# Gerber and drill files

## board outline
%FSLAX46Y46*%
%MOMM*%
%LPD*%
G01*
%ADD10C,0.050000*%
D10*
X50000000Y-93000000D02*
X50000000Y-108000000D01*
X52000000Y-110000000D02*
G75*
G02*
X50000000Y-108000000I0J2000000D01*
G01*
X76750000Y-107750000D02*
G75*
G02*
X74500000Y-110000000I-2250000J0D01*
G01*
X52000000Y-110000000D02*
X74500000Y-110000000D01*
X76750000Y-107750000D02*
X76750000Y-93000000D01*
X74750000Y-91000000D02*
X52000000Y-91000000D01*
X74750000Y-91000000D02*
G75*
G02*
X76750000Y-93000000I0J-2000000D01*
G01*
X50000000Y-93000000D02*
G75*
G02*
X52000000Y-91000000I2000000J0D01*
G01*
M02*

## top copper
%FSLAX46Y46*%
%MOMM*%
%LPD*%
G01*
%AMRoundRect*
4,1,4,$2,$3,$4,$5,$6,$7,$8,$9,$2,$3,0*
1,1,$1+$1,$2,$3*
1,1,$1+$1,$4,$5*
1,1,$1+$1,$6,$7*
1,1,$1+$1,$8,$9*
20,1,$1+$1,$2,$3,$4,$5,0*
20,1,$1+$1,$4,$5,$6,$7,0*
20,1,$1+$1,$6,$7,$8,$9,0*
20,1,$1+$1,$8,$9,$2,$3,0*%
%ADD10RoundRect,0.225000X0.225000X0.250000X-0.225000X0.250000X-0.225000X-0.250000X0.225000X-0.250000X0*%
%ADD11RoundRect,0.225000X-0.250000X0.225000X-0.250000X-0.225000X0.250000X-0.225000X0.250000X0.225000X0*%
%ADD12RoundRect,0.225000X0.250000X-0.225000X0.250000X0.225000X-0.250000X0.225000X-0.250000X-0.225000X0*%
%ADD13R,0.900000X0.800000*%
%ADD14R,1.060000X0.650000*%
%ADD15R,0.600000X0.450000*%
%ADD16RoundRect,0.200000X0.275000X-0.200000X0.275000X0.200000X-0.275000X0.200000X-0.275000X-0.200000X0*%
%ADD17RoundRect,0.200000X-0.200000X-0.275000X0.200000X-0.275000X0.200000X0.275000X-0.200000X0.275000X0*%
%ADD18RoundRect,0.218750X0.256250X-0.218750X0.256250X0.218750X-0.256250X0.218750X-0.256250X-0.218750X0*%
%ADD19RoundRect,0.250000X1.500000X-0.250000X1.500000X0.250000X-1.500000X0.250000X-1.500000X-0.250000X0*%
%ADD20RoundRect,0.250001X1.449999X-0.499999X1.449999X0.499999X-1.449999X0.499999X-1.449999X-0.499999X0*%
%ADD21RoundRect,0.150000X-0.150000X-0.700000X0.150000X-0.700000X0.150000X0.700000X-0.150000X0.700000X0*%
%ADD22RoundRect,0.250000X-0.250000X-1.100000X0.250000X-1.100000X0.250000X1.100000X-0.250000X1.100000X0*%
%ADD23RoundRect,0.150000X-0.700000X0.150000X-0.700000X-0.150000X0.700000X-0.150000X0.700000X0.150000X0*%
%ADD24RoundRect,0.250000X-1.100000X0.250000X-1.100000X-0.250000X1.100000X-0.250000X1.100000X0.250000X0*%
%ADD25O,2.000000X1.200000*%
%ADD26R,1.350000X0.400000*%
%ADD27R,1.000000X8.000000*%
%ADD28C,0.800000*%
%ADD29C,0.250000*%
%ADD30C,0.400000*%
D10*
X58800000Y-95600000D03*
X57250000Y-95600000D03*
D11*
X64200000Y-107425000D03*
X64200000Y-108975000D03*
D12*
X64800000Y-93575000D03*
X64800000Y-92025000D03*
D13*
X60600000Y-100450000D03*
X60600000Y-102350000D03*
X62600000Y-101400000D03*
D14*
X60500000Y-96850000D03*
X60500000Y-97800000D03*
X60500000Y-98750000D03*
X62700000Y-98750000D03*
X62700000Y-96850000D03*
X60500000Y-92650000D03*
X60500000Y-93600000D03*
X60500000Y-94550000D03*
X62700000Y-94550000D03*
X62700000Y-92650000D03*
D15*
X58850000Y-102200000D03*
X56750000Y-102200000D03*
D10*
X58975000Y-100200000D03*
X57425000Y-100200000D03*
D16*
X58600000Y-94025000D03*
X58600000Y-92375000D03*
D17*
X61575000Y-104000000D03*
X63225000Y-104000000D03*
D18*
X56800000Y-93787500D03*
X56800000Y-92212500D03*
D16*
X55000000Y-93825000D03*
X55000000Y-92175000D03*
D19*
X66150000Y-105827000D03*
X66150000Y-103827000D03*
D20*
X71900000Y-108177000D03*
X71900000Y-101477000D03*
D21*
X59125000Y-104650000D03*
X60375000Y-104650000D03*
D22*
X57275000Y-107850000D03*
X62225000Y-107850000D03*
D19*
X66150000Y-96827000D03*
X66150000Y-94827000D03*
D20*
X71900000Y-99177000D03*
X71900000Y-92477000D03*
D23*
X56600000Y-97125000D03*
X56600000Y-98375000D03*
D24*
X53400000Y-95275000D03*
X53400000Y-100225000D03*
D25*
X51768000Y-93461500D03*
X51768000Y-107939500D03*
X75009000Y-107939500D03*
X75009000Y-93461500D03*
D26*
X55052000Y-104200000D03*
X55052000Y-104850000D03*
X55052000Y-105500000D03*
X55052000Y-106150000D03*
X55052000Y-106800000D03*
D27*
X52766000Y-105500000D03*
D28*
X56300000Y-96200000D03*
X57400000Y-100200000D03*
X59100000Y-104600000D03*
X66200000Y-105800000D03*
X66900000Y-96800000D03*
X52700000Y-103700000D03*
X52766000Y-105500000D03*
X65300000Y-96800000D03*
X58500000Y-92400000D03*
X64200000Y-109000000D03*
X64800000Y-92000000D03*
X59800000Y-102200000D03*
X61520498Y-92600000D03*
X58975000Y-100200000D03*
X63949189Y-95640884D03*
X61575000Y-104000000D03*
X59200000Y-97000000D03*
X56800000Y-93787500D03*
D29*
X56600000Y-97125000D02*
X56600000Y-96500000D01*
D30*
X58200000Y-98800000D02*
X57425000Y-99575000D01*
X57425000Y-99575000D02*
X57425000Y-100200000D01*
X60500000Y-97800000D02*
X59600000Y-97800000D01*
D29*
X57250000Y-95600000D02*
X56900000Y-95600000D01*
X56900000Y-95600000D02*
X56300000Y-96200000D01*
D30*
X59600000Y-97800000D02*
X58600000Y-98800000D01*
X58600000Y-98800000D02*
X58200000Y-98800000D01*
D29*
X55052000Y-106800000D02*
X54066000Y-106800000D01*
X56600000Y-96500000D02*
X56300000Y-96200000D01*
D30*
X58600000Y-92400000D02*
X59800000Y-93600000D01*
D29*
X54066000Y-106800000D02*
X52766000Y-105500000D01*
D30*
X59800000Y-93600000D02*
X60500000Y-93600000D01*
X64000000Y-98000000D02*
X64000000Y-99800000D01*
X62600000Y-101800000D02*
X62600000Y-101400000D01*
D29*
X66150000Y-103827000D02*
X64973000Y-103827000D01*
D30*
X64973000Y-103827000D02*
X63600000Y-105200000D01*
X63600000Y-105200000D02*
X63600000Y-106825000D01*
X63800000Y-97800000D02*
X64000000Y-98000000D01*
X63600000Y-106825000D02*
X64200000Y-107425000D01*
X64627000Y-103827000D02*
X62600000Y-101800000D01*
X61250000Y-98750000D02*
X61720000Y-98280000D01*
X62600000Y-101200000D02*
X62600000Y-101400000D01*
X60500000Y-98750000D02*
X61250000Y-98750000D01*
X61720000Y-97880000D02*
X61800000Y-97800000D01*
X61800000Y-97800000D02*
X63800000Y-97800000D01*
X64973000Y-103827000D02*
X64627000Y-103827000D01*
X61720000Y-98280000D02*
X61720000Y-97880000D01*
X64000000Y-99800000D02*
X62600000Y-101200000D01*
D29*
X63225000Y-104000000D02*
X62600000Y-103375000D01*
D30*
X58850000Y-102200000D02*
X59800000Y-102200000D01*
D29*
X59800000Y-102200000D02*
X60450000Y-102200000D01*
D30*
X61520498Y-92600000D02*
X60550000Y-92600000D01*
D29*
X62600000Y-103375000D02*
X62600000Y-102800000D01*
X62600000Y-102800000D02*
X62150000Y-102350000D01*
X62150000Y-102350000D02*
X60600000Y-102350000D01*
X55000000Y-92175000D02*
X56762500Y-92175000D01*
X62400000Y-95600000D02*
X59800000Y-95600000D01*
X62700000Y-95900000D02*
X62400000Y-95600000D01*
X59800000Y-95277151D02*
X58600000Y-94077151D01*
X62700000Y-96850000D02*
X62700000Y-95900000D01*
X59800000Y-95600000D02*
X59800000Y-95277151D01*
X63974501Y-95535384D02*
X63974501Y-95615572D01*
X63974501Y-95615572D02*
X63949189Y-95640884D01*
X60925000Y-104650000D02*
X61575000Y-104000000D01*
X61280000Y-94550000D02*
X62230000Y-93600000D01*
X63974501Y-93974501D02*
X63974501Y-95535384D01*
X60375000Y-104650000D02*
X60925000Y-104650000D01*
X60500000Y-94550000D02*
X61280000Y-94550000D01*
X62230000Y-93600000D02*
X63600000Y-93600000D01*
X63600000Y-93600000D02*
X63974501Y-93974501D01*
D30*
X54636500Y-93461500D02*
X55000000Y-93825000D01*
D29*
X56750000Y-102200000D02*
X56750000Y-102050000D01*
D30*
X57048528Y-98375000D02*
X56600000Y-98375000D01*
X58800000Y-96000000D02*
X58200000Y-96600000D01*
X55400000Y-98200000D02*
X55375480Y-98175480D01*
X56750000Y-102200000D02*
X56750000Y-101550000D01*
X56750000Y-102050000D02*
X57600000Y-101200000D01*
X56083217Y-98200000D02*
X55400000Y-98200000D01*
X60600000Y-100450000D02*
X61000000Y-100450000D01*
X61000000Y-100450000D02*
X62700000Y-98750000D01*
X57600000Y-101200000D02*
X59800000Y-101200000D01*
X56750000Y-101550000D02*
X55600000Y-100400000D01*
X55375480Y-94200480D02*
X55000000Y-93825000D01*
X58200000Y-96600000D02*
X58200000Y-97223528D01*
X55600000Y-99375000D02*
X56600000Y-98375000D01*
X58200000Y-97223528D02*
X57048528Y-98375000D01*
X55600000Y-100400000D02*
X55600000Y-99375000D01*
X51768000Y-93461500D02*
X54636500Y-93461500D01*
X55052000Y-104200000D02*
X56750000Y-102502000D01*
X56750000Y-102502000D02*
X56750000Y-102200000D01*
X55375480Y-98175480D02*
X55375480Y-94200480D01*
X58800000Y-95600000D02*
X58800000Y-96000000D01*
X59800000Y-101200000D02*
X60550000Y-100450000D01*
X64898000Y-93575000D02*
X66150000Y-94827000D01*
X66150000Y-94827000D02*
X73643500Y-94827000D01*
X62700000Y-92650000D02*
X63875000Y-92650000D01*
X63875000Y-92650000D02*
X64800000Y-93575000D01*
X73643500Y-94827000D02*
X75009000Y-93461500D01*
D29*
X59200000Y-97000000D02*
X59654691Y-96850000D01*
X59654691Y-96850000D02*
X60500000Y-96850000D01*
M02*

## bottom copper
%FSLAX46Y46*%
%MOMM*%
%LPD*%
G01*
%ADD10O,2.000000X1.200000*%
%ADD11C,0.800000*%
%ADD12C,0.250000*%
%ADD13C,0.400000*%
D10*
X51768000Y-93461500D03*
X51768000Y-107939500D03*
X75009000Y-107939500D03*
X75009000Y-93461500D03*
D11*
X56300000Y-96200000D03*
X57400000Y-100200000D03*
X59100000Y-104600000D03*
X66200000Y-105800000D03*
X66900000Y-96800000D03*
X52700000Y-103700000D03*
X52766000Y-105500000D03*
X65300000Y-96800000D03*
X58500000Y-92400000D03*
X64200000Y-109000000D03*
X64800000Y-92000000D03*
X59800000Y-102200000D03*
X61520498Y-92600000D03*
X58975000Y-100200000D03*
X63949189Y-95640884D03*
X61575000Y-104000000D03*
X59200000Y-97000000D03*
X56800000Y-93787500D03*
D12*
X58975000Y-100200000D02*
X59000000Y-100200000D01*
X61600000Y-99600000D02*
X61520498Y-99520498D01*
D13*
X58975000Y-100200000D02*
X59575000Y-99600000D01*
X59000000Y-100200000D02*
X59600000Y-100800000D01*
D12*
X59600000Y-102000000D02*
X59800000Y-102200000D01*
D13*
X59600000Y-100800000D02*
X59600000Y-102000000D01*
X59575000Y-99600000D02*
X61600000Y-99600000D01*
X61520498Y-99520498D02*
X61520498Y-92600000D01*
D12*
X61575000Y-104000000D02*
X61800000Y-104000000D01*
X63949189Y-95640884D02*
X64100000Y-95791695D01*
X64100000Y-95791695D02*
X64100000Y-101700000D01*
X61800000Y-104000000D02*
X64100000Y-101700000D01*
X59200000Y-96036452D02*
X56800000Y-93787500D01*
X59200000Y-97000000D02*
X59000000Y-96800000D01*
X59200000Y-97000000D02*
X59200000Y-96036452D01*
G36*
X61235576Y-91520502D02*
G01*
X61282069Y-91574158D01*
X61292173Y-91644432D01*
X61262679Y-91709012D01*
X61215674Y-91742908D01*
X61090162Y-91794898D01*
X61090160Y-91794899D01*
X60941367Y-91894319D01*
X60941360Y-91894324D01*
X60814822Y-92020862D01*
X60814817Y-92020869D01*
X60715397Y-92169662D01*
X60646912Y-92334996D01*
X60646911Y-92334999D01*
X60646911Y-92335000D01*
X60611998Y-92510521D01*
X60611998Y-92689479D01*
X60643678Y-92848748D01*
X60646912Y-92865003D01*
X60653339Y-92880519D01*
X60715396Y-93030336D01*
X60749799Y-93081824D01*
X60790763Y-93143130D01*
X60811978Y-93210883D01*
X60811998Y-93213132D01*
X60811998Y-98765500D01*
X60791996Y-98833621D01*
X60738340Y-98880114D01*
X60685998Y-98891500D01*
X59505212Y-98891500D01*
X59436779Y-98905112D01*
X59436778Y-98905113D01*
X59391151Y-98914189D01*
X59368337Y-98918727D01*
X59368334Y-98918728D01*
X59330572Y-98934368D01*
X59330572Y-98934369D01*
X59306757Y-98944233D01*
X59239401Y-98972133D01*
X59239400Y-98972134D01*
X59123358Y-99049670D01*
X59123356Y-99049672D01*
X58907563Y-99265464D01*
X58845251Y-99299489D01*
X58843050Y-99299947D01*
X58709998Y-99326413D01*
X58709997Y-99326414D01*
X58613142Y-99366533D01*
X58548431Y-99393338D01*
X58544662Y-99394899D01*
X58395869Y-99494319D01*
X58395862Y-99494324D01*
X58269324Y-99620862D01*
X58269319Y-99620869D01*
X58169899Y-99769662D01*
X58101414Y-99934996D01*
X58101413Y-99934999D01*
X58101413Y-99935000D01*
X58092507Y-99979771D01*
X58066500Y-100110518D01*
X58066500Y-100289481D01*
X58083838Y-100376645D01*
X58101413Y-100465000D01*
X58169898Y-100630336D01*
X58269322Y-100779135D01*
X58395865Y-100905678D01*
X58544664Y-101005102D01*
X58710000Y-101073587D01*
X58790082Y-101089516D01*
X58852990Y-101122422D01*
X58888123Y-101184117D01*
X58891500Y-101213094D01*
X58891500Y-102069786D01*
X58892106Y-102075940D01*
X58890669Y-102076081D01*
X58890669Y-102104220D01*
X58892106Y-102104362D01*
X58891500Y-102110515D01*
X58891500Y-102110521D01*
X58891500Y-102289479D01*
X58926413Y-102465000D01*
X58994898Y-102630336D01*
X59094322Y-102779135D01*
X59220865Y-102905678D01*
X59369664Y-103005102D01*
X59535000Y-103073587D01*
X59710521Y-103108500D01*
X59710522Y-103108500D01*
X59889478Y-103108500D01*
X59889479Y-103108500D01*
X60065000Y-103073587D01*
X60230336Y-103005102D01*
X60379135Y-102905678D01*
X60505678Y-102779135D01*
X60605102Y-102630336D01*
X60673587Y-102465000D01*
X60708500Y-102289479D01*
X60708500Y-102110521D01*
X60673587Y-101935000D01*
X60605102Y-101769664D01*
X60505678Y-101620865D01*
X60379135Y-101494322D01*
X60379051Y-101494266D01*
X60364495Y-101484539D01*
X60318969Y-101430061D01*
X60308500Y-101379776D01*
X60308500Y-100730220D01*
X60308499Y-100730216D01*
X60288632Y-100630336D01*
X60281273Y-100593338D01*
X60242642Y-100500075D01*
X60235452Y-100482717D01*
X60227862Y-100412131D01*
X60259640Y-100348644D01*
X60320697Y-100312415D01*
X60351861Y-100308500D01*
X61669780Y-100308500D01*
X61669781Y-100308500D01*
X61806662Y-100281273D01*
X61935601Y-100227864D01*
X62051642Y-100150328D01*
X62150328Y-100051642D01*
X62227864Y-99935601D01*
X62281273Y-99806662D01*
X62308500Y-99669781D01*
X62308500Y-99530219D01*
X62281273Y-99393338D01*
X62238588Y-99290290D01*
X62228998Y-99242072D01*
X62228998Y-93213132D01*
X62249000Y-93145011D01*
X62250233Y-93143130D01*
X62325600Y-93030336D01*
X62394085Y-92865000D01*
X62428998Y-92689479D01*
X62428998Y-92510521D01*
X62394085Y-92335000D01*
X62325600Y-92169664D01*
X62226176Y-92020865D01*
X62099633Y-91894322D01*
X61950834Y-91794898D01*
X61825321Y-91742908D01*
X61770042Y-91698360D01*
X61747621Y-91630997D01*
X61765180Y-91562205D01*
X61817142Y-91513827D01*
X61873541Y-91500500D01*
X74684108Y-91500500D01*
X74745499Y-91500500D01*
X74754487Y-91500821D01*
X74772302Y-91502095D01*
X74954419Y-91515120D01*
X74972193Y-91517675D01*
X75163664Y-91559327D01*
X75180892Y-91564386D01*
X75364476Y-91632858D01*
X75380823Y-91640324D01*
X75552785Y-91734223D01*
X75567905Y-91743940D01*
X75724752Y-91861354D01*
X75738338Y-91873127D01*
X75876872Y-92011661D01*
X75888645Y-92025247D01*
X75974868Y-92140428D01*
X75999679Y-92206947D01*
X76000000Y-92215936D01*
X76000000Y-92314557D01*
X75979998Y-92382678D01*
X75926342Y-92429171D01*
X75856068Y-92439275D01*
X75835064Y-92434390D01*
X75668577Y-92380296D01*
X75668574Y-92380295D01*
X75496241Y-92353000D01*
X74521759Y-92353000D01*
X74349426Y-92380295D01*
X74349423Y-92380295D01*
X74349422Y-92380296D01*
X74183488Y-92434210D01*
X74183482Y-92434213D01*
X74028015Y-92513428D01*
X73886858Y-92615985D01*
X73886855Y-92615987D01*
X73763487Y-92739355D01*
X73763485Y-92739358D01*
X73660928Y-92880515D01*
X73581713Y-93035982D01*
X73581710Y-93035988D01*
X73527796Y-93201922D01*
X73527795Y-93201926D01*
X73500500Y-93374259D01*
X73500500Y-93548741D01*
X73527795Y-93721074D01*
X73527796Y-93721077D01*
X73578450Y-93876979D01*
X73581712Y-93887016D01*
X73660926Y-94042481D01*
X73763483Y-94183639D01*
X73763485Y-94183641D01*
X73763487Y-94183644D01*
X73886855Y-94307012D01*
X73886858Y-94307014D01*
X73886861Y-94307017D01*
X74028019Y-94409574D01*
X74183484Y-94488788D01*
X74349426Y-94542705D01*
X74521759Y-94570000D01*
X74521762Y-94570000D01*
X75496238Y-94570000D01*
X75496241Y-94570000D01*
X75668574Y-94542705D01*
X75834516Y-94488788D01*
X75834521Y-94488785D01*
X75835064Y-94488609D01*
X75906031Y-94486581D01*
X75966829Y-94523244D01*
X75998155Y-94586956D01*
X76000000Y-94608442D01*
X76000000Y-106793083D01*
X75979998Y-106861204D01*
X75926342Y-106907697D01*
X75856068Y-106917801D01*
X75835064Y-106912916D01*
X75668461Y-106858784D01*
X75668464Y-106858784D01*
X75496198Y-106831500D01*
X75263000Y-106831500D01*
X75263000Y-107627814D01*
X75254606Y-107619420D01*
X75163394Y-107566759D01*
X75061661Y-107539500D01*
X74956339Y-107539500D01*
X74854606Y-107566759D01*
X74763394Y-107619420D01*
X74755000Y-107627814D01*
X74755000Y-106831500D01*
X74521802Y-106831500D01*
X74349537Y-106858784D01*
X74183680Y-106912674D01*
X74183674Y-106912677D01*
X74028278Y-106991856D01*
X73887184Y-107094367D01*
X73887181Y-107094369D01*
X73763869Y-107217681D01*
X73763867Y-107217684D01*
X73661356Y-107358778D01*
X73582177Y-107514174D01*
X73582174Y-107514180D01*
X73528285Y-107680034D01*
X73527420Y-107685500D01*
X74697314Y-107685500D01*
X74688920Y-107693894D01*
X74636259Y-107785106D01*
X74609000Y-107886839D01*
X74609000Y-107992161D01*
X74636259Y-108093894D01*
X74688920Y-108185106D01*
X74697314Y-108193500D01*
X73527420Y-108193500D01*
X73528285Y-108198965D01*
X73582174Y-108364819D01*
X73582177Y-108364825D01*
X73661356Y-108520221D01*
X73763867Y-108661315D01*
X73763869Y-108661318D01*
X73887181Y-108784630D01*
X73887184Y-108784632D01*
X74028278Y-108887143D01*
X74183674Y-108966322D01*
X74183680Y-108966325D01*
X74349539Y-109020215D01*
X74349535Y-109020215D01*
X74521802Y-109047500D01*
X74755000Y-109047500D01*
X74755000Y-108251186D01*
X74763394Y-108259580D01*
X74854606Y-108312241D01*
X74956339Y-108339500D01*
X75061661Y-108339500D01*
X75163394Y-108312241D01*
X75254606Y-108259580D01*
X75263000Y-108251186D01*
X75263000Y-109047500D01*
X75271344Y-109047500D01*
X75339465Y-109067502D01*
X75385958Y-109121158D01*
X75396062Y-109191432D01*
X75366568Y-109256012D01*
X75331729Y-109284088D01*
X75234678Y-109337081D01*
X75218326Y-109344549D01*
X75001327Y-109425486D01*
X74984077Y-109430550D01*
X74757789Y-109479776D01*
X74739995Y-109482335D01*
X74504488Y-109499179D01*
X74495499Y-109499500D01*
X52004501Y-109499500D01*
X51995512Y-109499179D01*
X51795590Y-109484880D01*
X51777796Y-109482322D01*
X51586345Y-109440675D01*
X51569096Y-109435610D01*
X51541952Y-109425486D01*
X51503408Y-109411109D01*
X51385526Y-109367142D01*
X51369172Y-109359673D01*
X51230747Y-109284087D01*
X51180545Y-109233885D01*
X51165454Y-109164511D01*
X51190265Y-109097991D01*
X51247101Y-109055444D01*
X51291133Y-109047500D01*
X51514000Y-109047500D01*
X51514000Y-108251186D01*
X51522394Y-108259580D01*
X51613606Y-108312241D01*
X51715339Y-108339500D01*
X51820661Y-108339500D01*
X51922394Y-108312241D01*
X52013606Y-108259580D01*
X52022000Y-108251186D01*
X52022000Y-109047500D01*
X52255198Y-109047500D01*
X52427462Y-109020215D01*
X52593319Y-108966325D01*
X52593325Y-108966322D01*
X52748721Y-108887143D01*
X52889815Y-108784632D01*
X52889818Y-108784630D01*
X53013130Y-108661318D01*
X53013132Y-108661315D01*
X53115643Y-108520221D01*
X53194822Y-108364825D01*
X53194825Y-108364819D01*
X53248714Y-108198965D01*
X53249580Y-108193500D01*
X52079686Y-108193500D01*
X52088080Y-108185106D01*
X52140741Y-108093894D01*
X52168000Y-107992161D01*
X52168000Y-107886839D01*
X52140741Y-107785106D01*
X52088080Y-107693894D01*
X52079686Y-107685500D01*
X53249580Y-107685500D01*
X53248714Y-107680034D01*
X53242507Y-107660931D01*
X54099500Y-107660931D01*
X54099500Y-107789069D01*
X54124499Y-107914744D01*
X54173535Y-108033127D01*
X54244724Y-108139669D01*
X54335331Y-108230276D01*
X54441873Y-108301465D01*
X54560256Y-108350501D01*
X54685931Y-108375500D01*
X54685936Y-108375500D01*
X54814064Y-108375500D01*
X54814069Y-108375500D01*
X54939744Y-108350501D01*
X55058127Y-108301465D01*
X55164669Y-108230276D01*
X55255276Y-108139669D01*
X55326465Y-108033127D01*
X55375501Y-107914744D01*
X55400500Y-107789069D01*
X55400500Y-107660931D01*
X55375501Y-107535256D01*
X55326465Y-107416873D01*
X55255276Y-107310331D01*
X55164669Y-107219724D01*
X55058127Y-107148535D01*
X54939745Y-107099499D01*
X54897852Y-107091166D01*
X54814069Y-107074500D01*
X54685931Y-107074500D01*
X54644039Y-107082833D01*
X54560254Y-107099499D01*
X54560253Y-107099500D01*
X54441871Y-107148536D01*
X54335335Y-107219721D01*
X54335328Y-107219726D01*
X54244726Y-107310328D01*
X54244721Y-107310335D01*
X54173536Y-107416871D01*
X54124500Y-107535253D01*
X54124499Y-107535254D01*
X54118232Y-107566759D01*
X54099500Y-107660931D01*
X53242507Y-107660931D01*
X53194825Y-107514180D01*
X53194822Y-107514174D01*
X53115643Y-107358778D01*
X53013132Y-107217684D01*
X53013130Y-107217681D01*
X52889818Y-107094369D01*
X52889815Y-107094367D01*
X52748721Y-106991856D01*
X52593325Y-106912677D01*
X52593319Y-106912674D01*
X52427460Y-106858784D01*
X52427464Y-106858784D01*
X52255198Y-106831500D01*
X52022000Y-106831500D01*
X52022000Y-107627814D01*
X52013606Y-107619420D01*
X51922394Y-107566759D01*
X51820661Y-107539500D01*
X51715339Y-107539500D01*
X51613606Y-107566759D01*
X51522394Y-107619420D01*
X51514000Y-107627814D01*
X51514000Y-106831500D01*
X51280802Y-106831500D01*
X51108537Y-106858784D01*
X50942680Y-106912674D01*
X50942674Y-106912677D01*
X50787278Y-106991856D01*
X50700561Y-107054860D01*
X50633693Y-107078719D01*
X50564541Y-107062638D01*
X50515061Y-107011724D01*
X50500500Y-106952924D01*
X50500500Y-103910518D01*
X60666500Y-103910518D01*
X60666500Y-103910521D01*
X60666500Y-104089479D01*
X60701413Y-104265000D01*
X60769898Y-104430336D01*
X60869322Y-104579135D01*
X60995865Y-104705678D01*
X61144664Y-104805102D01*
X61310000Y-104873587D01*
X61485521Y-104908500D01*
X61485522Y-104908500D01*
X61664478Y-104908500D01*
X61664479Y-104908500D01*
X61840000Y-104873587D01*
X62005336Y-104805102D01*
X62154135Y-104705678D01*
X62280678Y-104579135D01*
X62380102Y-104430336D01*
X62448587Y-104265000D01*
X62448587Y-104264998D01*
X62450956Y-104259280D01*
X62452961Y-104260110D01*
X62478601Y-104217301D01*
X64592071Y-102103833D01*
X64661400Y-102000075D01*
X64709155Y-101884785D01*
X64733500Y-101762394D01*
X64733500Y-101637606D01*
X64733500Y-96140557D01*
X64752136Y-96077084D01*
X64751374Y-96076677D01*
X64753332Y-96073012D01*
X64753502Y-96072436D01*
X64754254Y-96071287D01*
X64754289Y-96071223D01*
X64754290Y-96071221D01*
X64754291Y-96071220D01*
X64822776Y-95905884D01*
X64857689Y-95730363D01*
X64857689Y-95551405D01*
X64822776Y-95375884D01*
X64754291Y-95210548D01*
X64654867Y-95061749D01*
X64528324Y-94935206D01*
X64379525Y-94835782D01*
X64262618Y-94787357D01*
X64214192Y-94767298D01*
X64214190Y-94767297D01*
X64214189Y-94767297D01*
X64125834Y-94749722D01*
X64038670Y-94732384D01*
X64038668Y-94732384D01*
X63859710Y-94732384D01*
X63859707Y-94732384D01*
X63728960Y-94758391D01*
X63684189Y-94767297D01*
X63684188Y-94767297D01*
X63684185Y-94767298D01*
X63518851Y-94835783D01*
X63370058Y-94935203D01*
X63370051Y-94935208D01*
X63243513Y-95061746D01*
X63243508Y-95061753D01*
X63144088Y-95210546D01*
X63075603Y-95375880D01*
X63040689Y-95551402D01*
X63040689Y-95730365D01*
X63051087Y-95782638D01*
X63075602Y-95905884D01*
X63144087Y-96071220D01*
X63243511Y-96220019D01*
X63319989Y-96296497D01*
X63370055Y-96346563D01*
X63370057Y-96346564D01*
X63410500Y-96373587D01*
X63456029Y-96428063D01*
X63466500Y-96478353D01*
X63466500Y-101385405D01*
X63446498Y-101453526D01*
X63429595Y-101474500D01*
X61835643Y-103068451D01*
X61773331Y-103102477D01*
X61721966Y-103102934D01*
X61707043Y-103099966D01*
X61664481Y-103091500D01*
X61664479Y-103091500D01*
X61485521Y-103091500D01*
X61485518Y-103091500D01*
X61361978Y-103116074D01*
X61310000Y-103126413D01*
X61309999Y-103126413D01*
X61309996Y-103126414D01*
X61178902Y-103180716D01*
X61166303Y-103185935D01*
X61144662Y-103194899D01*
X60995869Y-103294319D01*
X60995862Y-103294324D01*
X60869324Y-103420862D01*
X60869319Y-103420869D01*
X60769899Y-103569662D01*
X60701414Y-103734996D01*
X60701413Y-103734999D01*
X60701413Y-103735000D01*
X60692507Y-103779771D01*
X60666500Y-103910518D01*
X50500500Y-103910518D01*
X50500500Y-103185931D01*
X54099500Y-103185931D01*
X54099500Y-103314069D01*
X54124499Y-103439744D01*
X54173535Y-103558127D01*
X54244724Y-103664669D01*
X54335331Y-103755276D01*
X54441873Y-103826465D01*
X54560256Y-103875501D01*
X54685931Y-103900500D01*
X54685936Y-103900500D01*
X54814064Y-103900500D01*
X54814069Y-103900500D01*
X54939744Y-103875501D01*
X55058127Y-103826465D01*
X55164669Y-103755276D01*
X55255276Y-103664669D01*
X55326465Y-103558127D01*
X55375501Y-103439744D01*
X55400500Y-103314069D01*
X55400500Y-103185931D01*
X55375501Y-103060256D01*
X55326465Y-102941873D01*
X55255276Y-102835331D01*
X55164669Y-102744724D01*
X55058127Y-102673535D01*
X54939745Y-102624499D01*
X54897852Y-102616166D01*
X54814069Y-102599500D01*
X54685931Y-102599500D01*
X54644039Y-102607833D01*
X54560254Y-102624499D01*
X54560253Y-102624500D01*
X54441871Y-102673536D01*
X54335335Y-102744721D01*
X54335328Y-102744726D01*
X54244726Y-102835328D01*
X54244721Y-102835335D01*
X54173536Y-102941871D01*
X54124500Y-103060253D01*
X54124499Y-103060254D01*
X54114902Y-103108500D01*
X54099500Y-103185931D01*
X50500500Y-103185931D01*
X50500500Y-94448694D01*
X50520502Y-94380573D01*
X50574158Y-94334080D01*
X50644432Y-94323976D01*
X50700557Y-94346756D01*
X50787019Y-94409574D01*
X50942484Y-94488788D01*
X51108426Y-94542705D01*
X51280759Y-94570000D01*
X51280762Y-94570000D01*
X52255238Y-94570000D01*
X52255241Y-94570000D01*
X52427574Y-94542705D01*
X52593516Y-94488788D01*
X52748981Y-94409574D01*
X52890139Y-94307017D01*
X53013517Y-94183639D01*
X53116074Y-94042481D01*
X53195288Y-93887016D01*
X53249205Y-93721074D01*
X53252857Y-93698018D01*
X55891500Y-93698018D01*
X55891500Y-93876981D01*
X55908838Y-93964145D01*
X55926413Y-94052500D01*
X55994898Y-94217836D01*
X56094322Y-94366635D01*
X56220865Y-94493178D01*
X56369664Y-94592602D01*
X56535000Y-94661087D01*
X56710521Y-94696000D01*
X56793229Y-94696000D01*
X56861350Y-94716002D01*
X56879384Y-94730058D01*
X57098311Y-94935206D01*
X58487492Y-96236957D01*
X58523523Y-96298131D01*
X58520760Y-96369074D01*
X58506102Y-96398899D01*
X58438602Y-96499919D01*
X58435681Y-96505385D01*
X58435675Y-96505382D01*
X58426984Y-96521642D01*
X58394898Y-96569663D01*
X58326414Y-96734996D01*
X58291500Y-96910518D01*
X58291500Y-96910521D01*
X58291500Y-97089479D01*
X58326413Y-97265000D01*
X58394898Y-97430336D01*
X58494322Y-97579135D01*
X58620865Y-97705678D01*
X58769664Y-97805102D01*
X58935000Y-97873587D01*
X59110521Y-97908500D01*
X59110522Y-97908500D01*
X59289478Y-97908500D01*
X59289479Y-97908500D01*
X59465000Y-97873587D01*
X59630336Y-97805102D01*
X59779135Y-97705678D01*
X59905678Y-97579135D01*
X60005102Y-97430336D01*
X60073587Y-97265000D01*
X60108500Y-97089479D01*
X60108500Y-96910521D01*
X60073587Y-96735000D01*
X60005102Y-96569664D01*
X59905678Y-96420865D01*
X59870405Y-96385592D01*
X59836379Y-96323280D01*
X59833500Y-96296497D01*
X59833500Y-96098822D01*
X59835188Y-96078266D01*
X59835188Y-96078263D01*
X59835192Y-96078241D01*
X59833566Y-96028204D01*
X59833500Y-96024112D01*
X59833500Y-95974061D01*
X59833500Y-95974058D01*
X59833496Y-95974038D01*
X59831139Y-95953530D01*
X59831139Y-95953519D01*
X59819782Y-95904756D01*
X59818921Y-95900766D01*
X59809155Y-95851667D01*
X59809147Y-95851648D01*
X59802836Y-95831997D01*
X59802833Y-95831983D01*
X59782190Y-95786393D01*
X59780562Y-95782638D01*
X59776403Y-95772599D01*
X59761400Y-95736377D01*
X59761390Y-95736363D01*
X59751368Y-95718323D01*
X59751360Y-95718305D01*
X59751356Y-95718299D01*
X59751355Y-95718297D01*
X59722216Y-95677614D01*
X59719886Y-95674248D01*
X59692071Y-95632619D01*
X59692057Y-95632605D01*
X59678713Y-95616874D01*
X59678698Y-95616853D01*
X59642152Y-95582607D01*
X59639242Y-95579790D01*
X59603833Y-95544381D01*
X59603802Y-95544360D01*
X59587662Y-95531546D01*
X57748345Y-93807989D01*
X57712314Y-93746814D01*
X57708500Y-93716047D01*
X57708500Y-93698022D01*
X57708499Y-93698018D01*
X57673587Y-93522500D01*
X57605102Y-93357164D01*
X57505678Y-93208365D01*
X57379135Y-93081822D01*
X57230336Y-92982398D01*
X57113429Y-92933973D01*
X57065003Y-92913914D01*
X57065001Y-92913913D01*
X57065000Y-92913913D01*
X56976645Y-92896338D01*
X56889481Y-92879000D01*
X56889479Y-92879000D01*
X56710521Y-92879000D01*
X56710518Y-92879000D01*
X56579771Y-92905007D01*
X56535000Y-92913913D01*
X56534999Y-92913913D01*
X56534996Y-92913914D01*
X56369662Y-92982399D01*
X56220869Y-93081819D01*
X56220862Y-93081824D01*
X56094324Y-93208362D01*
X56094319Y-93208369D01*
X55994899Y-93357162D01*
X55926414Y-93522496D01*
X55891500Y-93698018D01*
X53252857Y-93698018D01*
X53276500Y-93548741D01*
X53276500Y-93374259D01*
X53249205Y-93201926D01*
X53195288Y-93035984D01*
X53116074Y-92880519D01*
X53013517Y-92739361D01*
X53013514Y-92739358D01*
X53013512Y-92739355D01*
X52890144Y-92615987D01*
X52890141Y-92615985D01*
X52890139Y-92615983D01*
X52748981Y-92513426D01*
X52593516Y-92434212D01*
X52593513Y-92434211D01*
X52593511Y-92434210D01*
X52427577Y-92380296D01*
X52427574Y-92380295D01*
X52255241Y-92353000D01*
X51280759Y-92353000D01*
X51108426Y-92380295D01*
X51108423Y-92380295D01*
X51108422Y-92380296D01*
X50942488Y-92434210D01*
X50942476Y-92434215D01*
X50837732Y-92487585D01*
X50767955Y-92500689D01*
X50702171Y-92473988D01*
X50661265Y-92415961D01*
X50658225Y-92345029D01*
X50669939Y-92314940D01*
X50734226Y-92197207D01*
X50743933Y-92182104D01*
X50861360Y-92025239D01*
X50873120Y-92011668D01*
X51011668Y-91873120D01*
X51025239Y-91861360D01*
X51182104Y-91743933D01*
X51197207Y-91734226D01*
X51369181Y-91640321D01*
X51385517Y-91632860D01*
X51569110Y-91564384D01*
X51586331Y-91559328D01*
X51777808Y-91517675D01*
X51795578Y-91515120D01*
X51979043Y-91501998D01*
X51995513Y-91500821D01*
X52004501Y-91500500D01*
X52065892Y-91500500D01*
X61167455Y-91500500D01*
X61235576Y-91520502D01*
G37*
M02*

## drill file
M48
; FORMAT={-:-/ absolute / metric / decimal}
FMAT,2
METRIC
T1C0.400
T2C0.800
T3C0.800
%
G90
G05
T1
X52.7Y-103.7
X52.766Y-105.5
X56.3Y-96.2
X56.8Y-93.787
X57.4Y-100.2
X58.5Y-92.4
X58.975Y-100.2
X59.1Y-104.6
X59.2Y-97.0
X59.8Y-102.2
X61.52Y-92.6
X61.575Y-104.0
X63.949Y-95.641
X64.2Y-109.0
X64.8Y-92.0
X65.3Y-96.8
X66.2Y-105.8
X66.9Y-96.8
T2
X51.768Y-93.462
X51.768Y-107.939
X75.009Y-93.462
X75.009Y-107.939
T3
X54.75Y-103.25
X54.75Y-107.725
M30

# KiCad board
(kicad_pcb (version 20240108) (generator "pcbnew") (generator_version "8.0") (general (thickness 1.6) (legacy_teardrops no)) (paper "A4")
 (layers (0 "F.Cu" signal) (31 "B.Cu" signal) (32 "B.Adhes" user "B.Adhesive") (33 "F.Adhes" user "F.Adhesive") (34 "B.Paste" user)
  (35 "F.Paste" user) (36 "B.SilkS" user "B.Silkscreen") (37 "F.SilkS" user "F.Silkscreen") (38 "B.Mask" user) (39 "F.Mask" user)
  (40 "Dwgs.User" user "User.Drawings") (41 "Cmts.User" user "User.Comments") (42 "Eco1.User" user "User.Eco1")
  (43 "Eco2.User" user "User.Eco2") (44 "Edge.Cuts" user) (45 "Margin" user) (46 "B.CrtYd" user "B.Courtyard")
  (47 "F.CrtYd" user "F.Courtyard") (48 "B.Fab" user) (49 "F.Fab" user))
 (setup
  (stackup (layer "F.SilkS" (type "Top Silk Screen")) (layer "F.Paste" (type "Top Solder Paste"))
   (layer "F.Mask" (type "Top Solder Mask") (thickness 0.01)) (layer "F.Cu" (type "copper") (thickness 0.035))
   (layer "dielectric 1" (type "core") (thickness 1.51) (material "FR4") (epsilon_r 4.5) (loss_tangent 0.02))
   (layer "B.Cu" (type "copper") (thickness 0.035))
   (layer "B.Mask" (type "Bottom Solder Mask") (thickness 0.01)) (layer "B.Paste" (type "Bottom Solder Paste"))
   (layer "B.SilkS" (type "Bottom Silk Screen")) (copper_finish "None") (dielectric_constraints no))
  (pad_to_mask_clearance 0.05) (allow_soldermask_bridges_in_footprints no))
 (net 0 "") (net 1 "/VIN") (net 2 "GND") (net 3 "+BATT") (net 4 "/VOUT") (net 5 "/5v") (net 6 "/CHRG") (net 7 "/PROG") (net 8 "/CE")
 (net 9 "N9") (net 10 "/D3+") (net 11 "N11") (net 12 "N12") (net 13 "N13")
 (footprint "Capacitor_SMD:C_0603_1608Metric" (layer "F.Cu") (at 58.025 95.6 180)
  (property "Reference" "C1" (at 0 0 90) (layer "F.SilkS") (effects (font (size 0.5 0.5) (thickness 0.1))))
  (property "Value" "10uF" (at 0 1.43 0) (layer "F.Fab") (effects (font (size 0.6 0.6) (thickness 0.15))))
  (pad "1" smd roundrect (at -0.775 0 180) (size 0.9 0.95) (layers "F.Cu" "F.Paste" "F.Mask") (roundrect_rratio 0.25) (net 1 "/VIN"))
  (pad "2" smd roundrect (at 0.775 0 180) (size 0.9 0.95) (layers "F.Cu" "F.Paste" "F.Mask") (roundrect_rratio 0.25) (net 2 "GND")))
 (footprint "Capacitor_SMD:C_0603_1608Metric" (layer "F.Cu") (at 64.2 108.2 -90)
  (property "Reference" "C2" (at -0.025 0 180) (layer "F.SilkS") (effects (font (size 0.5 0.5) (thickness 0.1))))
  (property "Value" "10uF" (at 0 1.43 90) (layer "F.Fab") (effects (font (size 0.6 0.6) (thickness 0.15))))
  (pad "1" smd roundrect (at -0.775 0 270) (size 0.9 0.95) (layers "F.Cu" "F.Paste" "F.Mask") (roundrect_rratio 0.25) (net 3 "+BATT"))
  (pad "2" smd roundrect (at 0.775 0 270) (size 0.9 0.95) (layers "F.Cu" "F.Paste" "F.Mask") (roundrect_rratio 0.25) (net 2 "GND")))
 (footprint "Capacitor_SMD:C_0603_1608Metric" (layer "F.Cu") (at 64.8 92.8 90)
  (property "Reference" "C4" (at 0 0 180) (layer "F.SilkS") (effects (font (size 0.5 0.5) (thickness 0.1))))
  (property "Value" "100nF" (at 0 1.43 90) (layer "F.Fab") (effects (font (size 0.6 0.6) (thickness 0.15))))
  (pad "1" smd roundrect (at -0.775 0 90) (size 0.9 0.95) (layers "F.Cu" "F.Paste" "F.Mask") (roundrect_rratio 0.25) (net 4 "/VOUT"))
  (pad "2" smd roundrect (at 0.775 0 90) (size 0.9 0.95) (layers "F.Cu" "F.Paste" "F.Mask") (roundrect_rratio 0.25) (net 2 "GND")))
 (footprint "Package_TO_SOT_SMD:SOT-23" (layer "F.Cu") (at 61.6 101.4)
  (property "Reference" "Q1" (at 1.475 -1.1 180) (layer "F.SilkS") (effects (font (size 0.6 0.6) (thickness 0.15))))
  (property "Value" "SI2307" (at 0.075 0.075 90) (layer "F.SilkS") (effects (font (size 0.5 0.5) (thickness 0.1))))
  (pad "1" smd rect (at -1 -0.95) (size 0.9 0.8) (layers "F.Cu" "F.Paste" "F.Mask") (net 1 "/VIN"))
  (pad "2" smd rect (at -1 0.95) (size 0.9 0.8) (layers "F.Cu" "F.Paste" "F.Mask") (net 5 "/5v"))
  (pad "3" smd rect (at 1 0) (size 0.9 0.8) (layers "F.Cu" "F.Paste" "F.Mask") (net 3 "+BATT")))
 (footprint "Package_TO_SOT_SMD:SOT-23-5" (layer "F.Cu") (at 61.6 97.8)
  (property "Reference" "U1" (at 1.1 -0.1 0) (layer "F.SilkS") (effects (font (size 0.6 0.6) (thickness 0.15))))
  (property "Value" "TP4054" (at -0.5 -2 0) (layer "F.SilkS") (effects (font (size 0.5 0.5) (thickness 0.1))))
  (pad "1" smd rect (at -1.1 -0.95) (size 1.06 0.65) (layers "F.Cu" "F.Paste" "F.Mask") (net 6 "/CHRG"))
  (pad "2" smd rect (at -1.1 0) (size 1.06 0.65) (layers "F.Cu" "F.Paste" "F.Mask") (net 2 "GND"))
  (pad "3" smd rect (at -1.1 0.95) (size 1.06 0.65) (layers "F.Cu" "F.Paste" "F.Mask") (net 3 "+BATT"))
  (pad "4" smd rect (at 1.1 0.95) (size 1.06 0.65) (layers "F.Cu" "F.Paste" "F.Mask") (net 1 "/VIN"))
  (pad "5" smd rect (at 1.1 -0.95) (size 1.06 0.65) (layers "F.Cu" "F.Paste" "F.Mask") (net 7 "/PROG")))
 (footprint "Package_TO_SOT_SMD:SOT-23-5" (layer "F.Cu") (at 61.6 93.6)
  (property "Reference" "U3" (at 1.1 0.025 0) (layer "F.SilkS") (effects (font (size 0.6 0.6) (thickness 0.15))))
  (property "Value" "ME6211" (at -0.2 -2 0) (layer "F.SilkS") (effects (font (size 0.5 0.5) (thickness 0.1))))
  (pad "1" smd rect (at -1.1 -0.95) (size 1.06 0.65) (layers "F.Cu" "F.Paste" "F.Mask") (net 5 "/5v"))
  (pad "2" smd rect (at -1.1 0) (size 1.06 0.65) (layers "F.Cu" "F.Paste" "F.Mask") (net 2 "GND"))
  (pad "3" smd rect (at -1.1 0.95) (size 1.06 0.65) (layers "F.Cu" "F.Paste" "F.Mask") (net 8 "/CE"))
  (pad "4" smd rect (at 1.1 0.95) (size 1.06 0.65) (layers "F.Cu" "F.Paste" "F.Mask") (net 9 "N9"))
  (pad "5" smd rect (at 1.1 -0.95) (size 1.06 0.65) (layers "F.Cu" "F.Paste" "F.Mask") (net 4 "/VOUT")))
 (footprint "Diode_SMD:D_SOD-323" (layer "F.Cu") (at 57.8 102.2 180)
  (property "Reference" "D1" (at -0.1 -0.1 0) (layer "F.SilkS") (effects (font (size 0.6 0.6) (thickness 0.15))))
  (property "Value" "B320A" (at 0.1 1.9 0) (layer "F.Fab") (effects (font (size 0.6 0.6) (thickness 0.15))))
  (pad "1" smd rect (at -1.05 0 180) (size 0.6 0.45) (layers "F.Cu" "F.Paste" "F.Mask") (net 5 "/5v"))
  (pad "2" smd rect (at 1.05 0 180) (size 0.6 0.45) (layers "F.Cu" "F.Paste" "F.Mask") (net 1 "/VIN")))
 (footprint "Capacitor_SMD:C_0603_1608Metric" (layer "F.Cu") (at 58.2 100.2 180)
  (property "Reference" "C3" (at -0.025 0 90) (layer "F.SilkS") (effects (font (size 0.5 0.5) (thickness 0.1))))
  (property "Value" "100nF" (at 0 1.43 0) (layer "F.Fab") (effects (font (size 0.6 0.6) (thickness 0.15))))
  (pad "1" smd roundrect (at -0.775 0 180) (size 0.9 0.95) (layers "F.Cu" "F.Paste" "F.Mask") (roundrect_rratio 0.25) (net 5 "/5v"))
  (pad "2" smd roundrect (at 0.775 0 180) (size 0.9 0.95) (layers "F.Cu" "F.Paste" "F.Mask") (roundrect_rratio 0.25) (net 2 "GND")))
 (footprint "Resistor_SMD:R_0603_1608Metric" (layer "F.Cu") (at 58.6 93.2 90)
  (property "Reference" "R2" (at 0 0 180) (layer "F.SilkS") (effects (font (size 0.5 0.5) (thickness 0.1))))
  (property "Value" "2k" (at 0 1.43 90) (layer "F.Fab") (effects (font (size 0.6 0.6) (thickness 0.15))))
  (pad "1" smd roundrect (at -0.825 0 90) (size 0.8 0.95) (layers "F.Cu" "F.Paste" "F.Mask") (roundrect_rratio 0.25) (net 7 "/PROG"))
  (pad "2" smd roundrect (at 0.825 0 90) (size 0.8 0.95) (layers "F.Cu" "F.Paste" "F.Mask") (roundrect_rratio 0.25) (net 2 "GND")))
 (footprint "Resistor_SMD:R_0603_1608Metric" (layer "F.Cu") (at 62.4 104)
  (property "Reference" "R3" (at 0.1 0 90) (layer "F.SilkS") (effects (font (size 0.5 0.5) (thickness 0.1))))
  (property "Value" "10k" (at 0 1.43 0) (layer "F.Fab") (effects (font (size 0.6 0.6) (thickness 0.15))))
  (pad "1" smd roundrect (at -0.825 0) (size 0.8 0.95) (layers "F.Cu" "F.Paste" "F.Mask") (roundrect_rratio 0.25) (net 8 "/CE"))
  (pad "2" smd roundrect (at 0.825 0) (size 0.8 0.95) (layers "F.Cu" "F.Paste" "F.Mask") (roundrect_rratio 0.25) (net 5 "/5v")))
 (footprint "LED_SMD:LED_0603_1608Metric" (layer "F.Cu") (at 56.8 93 90)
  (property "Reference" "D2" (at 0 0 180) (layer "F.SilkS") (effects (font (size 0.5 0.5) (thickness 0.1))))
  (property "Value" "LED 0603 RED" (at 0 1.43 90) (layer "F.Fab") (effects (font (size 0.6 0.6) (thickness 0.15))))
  (pad "1" smd roundrect (at -0.7875 0 90) (size 0.875 0.95) (layers "F.Cu" "F.Paste" "F.Mask") (roundrect_rratio 0.25) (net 6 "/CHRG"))
  (pad "2" smd roundrect (at 0.7875 0 90) (size 0.875 0.95) (layers "F.Cu" "F.Paste" "F.Mask") (roundrect_rratio 0.25) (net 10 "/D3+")))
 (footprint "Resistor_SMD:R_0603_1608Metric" (layer "F.Cu") (at 55 93 90)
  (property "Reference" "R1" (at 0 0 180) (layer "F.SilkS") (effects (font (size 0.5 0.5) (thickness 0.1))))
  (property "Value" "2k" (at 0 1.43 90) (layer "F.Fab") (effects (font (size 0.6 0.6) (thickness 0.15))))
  (pad "1" smd roundrect (at -0.825 0 90) (size 0.8 0.95) (layers "F.Cu" "F.Paste" "F.Mask") (roundrect_rratio 0.25) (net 1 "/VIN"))
  (pad "2" smd roundrect (at 0.825 0 90) (size 0.8 0.95) (layers "F.Cu" "F.Paste" "F.Mask") (roundrect_rratio 0.25) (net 10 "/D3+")))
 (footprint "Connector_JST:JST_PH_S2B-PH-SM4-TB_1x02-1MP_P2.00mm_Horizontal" (layer "F.Cu") (at 69 104.827 90)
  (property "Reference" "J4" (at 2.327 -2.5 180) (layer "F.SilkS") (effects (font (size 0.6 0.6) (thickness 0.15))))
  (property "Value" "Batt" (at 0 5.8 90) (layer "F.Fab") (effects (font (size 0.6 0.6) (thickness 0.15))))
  (pad "1" smd roundrect (at -1 -2.85 90) (size 1 3.5) (layers "F.Cu" "F.Paste" "F.Mask") (roundrect_rratio 0.25) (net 2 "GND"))
  (pad "2" smd roundrect (at 1 -2.85 90) (size 1 3.5) (layers "F.Cu" "F.Paste" "F.Mask") (roundrect_rratio 0.25) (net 3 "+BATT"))
  (pad "MP" smd roundrect (at -3.35 2.9 90) (size 1.5 3.4) (layers "F.Cu" "F.Paste" "F.Mask") (roundrect_rratio 0.1666673333))
  (pad "MP" smd roundrect (at 3.35 2.9 90) (size 1.5 3.4) (layers "F.Cu" "F.Paste" "F.Mask") (roundrect_rratio 0.1666673333)))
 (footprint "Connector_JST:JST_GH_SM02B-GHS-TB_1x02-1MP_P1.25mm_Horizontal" (layer "F.Cu") (at 59.75 106.5)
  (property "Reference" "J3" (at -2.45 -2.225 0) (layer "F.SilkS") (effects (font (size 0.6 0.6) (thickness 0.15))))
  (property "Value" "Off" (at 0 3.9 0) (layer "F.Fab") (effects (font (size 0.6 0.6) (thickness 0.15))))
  (pad "1" smd roundrect (at -0.625 -1.85) (size 0.6 1.7) (layers "F.Cu" "F.Paste" "F.Mask") (roundrect_rratio 0.25) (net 2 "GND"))
  (pad "2" smd roundrect (at 0.625 -1.85) (size 0.6 1.7) (layers "F.Cu" "F.Paste" "F.Mask") (roundrect_rratio 0.25) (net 8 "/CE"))
  (pad "MP" smd roundrect (at -2.475 1.35) (size 1 2.7) (layers "F.Cu" "F.Paste" "F.Mask") (roundrect_rratio 0.25))
  (pad "MP" smd roundrect (at 2.475 1.35) (size 1 2.7) (layers "F.Cu" "F.Paste" "F.Mask") (roundrect_rratio 0.25)))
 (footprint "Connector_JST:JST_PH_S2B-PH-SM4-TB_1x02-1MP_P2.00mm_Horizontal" (layer "F.Cu") (at 69 95.827 90)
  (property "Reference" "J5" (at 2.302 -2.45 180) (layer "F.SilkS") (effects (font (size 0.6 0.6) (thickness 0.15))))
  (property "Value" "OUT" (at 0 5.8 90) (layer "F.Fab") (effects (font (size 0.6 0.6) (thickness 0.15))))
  (pad "1" smd roundrect (at -1 -2.85 90) (size 1 3.5) (layers "F.Cu" "F.Paste" "F.Mask") (roundrect_rratio 0.25) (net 2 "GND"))
  (pad "2" smd roundrect (at 1 -2.85 90) (size 1 3.5) (layers "F.Cu" "F.Paste" "F.Mask") (roundrect_rratio 0.25) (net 4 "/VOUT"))
  (pad "MP" smd roundrect (at -3.35 2.9 90) (size 1.5 3.4) (layers "F.Cu" "F.Paste" "F.Mask") (roundrect_rratio 0.1666673333))
  (pad "MP" smd roundrect (at 3.35 2.9 90) (size 1.5 3.4) (layers "F.Cu" "F.Paste" "F.Mask") (roundrect_rratio 0.1666673333)))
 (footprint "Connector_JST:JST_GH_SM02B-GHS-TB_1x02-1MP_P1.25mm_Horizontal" (layer "F.Cu") (at 54.75 97.75 -90)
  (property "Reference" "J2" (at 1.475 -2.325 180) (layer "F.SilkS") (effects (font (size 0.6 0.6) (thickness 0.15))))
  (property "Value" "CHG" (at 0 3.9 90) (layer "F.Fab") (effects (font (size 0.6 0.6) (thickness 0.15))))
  (pad "1" smd roundrect (at -0.625 -1.85 270) (size 0.6 1.7) (layers "F.Cu" "F.Paste" "F.Mask") (roundrect_rratio 0.25) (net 2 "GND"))
  (pad "2" smd roundrect (at 0.625 -1.85 270) (size 0.6 1.7) (layers "F.Cu" "F.Paste" "F.Mask") (roundrect_rratio 0.25) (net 1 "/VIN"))
  (pad "MP" smd roundrect (at -2.475 1.35 270) (size 1 2.7) (layers "F.Cu" "F.Paste" "F.Mask") (roundrect_rratio 0.25))
  (pad "MP" smd roundrect (at 2.475 1.35 270) (size 1 2.7) (layers "F.Cu" "F.Paste" "F.Mask") (roundrect_rratio 0.25)))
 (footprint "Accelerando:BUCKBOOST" (layer "F.Cu") (at 50.244 91.1755)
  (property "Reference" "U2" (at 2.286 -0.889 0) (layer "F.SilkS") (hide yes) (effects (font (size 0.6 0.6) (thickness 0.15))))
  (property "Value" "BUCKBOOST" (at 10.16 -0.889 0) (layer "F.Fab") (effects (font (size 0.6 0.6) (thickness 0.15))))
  (pad "1" thru_hole oval (at 1.524 2.286 270) (size 1.2 2) (drill 0.8) (layers "*.Cu" "*.Mask") (remove_unused_layers no) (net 1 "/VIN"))
  (pad "2" thru_hole oval (at 1.524 16.764 270) (size 1.2 2) (drill 0.8) (layers "*.Cu" "*.Mask") (remove_unused_layers no) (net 2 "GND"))
  (pad "3" thru_hole oval (at 24.765 16.764 90) (size 1.2 2) (drill 0.8) (layers "*.Cu" "*.Mask") (remove_unused_layers no) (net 2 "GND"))
  (pad "4" thru_hole oval (at 24.765 2.286 90) (size 1.2 2) (drill 0.8) (layers "*.Cu" "*.Mask") (remove_unused_layers no) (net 4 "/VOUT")))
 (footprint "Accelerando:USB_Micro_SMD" (layer "F.Cu") (at 51.75 105.5 -90)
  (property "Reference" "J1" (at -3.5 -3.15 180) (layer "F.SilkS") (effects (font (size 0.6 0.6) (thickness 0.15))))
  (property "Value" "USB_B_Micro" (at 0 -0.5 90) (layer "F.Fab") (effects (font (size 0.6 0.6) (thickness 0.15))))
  (pad "" np_thru_hole circle (at -2.25 -3 270) (size 0.8 0.8) (drill 0.8) (layers "*.Cu" "*.Mask"))
  (pad "" np_thru_hole circle (at 2.225 -3 270) (size 0.8 0.8) (drill 0.8) (layers "*.Cu" "*.Mask"))
  (pad "1" smd rect (at -1.3 -3.302 270) (size 0.4 1.35) (layers "F.Cu" "F.Paste" "F.Mask") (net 1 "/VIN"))
  (pad "2" smd rect (at -0.65 -3.302 270) (size 0.4 1.35) (layers "F.Cu" "F.Paste" "F.Mask") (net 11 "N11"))
  (pad "3" smd rect (at 0 -3.302 270) (size 0.4 1.35) (layers "F.Cu" "F.Paste" "F.Mask") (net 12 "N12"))
  (pad "4" smd rect (at 0.65 -3.302 270) (size 0.4 1.35) (layers "F.Cu" "F.Paste" "F.Mask") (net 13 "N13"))
  (pad "5" smd rect (at 1.3 -3.302 270) (size 0.4 1.35) (layers "F.Cu" "F.Paste" "F.Mask") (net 2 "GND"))
  (pad "6" smd rect (at 0 -1.016 270) (size 8 1) (layers "F.Cu" "F.Paste" "F.Mask") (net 2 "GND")))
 (gr_line (start 50 93) (end 50 108) (stroke (width 0.05) (type solid)) (layer "Edge.Cuts"))
 (gr_arc (start 52 110) (mid 50.585786 109.414214) (end 50 108) (stroke (width 0.05) (type solid)) (layer "Edge.Cuts"))
 (gr_arc (start 76.75 107.75) (mid 76.09099 109.34099) (end 74.5 110) (stroke (width 0.05) (type solid)) (layer "Edge.Cuts"))
 (gr_line (start 52 110) (end 74.5 110) (stroke (width 0.05) (type solid)) (layer "Edge.Cuts"))
 (gr_line (start 76.75 107.75) (end 76.75 93) (stroke (width 0.05) (type solid)) (layer "Edge.Cuts"))
 (gr_line (start 74.75 91) (end 52 91) (stroke (width 0.05) (type solid)) (layer "Edge.Cuts"))
 (gr_arc (start 74.75 91) (mid 76.164214 91.585786) (end 76.75 93) (stroke (width 0.05) (type solid)) (layer "Edge.Cuts"))
 (gr_arc (start 50 93) (mid 50.585786 91.585786) (end 52 91) (stroke (width 0.05) (type solid)) (layer "Edge.Cuts"))
 (segment (start 56.6 97.125) (end 56.6 96.5) (width 0.25) (layer "F.Cu") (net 2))
 (segment (start 58.2 98.8) (end 57.425 99.575) (width 0.4) (layer "F.Cu") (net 2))
 (segment (start 57.425 99.575) (end 57.425 100.2) (width 0.4) (layer "F.Cu") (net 2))
 (segment (start 60.5 97.8) (end 59.6 97.8) (width 0.4) (layer "F.Cu") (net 2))
 (segment (start 57.25 95.6) (end 56.9 95.6) (width 0.25) (layer "F.Cu") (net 2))
 (segment (start 56.9 95.6) (end 56.3 96.2) (width 0.25) (layer "F.Cu") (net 2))
 (segment (start 59.6 97.8) (end 58.6 98.8) (width 0.4) (layer "F.Cu") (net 2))
 (segment (start 58.6 98.8) (end 58.2 98.8) (width 0.4) (layer "F.Cu") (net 2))
 (segment (start 55.052 106.8) (end 54.066 106.8) (width 0.25) (layer "F.Cu") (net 2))
 (segment (start 56.6 96.5) (end 56.3 96.2) (width 0.25) (layer "F.Cu") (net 2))
 (segment (start 58.6 92.4) (end 59.8 93.6) (width 0.4) (layer "F.Cu") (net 2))
 (segment (start 54.066 106.8) (end 52.766 105.5) (width 0.25) (layer "F.Cu") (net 2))
 (segment (start 59.8 93.6) (end 60.5 93.6) (width 0.4) (layer "F.Cu") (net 2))
 (via (at 56.3 96.2) (size 0.8) (drill 0.4) (layers "F.Cu" "B.Cu") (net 2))
 (via (at 57.4 100.2) (size 0.8) (drill 0.4) (layers "F.Cu" "B.Cu") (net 2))
 (via (at 59.1 104.6) (size 0.8) (drill 0.4) (layers "F.Cu" "B.Cu") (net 2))
 (via (at 66.2 105.8) (size 0.8) (drill 0.4) (layers "F.Cu" "B.Cu") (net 2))
 (via (at 66.9 96.8) (size 0.8) (drill 0.4) (layers "F.Cu" "B.Cu") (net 2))
 (via (at 52.7 103.7) (size 0.8) (drill 0.4) (layers "F.Cu" "B.Cu") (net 2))
 (via (at 52.766 105.5) (size 0.8) (drill 0.4) (layers "F.Cu" "B.Cu") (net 2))
 (via (at 65.3 96.8) (size 0.8) (drill 0.4) (layers "F.Cu" "B.Cu") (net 2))
 (via (at 58.5 92.4) (size 0.8) (drill 0.4) (layers "F.Cu" "B.Cu") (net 2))
 (via (at 64.2 109) (size 0.8) (drill 0.4) (layers "F.Cu" "B.Cu") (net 2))
 (via (at 64.8 92) (size 0.8) (drill 0.4) (layers "F.Cu" "B.Cu") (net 2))
 (segment (start 64 98) (end 64 99.8) (width 0.4) (layer "F.Cu") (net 3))
 (segment (start 62.6 101.8) (end 62.6 101.4) (width 0.4) (layer "F.Cu") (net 3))
 (segment (start 66.15 103.827) (end 64.973 103.827) (width 0.25) (layer "F.Cu") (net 3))
 (segment (start 64.973 103.827) (end 63.6 105.2) (width 0.4) (layer "F.Cu") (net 3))
 (segment (start 63.6 105.2) (end 63.6 106.825) (width 0.4) (layer "F.Cu") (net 3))
 (segment (start 63.8 97.8) (end 64 98) (width 0.4) (layer "F.Cu") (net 3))
 (segment (start 63.6 106.825) (end 64.2 107.425) (width 0.4) (layer "F.Cu") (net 3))
 (segment (start 64.627 103.827) (end 62.6 101.8) (width 0.4) (layer "F.Cu") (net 3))
 (segment (start 61.25 98.75) (end 61.72 98.28) (width 0.4) (layer "F.Cu") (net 3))
 (segment (start 62.6 101.2) (end 62.6 101.4) (width 0.4) (layer "F.Cu") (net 3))
 (segment (start 60.5 98.75) (end 61.25 98.75) (width 0.4) (layer "F.Cu") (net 3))
 (segment (start 61.72 97.88) (end 61.8 97.8) (width 0.4) (layer "F.Cu") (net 3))
 (segment (start 61.8 97.8) (end 63.8 97.8) (width 0.4) (layer "F.Cu") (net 3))
 (segment (start 64.973 103.827) (end 64.627 103.827) (width 0.4) (layer "F.Cu") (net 3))
 (segment (start 61.72 98.28) (end 61.72 97.88) (width 0.4) (layer "F.Cu") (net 3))
 (segment (start 64 99.8) (end 62.6 101.2) (width 0.4) (layer "F.Cu") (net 3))
 (segment (start 63.225 104) (end 62.6 103.375) (width 0.25) (layer "F.Cu") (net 5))
 (segment (start 58.85 102.2) (end 59.8 102.2) (width 0.4) (layer "F.Cu") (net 5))
 (segment (start 59.8 102.2) (end 60.45 102.2) (width 0.25) (layer "F.Cu") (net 5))
 (segment (start 61.520498 92.6) (end 60.55 92.6) (width 0.4) (layer "F.Cu") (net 5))
 (segment (start 62.6 103.375) (end 62.6 102.8) (width 0.25) (layer "F.Cu") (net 5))
 (segment (start 62.6 102.8) (end 62.15 102.35) (width 0.25) (layer "F.Cu") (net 5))
 (segment (start 62.15 102.35) (end 60.6 102.35) (width 0.25) (layer "F.Cu") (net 5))
 (via (at 59.8 102.2) (size 0.8) (drill 0.4) (layers "F.Cu" "B.Cu") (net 5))
 (via (at 61.520498 92.6) (size 0.8) (drill 0.4) (layers "F.Cu" "B.Cu") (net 5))
 (via (at 58.975 100.2) (size 0.8) (drill 0.4) (layers "F.Cu" "B.Cu") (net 5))
 (segment (start 58.975 100.2) (end 59 100.2) (width 0.25) (layer "B.Cu") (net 5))
 (segment (start 61.6 99.6) (end 61.520498 99.520498) (width 0.25) (layer "B.Cu") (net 5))
 (segment (start 58.975 100.2) (end 59.575 99.6) (width 0.4) (layer "B.Cu") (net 5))
 (segment (start 59 100.2) (end 59.6 100.8) (width 0.4) (layer "B.Cu") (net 5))
 (segment (start 59.6 102) (end 59.8 102.2) (width 0.25) (layer "B.Cu") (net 5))
 (segment (start 59.6 100.8) (end 59.6 102) (width 0.4) (layer "B.Cu") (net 5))
 (segment (start 59.575 99.6) (end 61.6 99.6) (width 0.4) (layer "B.Cu") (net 5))
 (segment (start 61.520498 99.520498) (end 61.520498 92.6) (width 0.4) (layer "B.Cu") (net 5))
 (segment (start 55 92.175) (end 56.7625 92.175) (width 0.25) (layer "F.Cu") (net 10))
 (segment (start 62.4 95.6) (end 59.8 95.6) (width 0.25) (layer "F.Cu") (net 7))
 (segment (start 62.7 95.9) (end 62.4 95.6) (width 0.25) (layer "F.Cu") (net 7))
 (segment (start 59.8 95.277151) (end 58.6 94.077151) (width 0.25) (layer "F.Cu") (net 7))
 (segment (start 62.7 96.85) (end 62.7 95.9) (width 0.25) (layer "F.Cu") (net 7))
 (segment (start 59.8 95.6) (end 59.8 95.277151) (width 0.25) (layer "F.Cu") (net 7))
 (segment (start 63.974501 95.535384) (end 63.974501 95.615572) (width 0.25) (layer "F.Cu") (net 8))
 (segment (start 63.974501 95.615572) (end 63.949189 95.640884) (width 0.25) (layer "F.Cu") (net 8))
 (segment (start 60.925 104.65) (end 61.575 104) (width 0.25) (layer "F.Cu") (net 8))
 (segment (start 61.28 94.55) (end 62.23 93.6) (width 0.25) (layer "F.Cu") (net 8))
 (segment (start 63.974501 93.974501) (end 63.974501 95.535384) (width 0.25) (layer "F.Cu") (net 8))
 (segment (start 60.375 104.65) (end 60.925 104.65) (width 0.25) (layer "F.Cu") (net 8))
 (segment (start 60.5 94.55) (end 61.28 94.55) (width 0.25) (layer "F.Cu") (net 8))
 (segment (start 62.23 93.6) (end 63.6 93.6) (width 0.25) (layer "F.Cu") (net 8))
 (segment (start 63.6 93.6) (end 63.974501 93.974501) (width 0.25) (layer "F.Cu") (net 8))
 (via (at 63.949189 95.640884) (size 0.8) (drill 0.4) (layers "F.Cu" "B.Cu") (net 8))
 (via (at 61.575 104) (size 0.8) (drill 0.4) (layers "F.Cu" "B.Cu") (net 8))
 (segment (start 61.575 104) (end 61.8 104) (width 0.25) (layer "B.Cu") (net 8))
 (segment (start 63.949189 95.640884) (end 64.1 95.791695) (width 0.25) (layer "B.Cu") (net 8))
 (segment (start 64.1 95.791695) (end 64.1 101.7) (width 0.25) (layer "B.Cu") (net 8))
 (segment (start 61.8 104) (end 64.1 101.7) (width 0.25) (layer "B.Cu") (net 8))
 (segment (start 54.6365 93.4615) (end 55 93.825) (width 0.4) (layer "F.Cu") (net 1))
 (segment (start 56.75 102.2) (end 56.75 102.05) (width 0.25) (layer "F.Cu") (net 1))
 (segment (start 57.048528 98.375) (end 56.6 98.375) (width 0.4) (layer "F.Cu") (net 1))
 (segment (start 58.8 96) (end 58.2 96.6) (width 0.4) (layer "F.Cu") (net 1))
 (segment (start 55.4 98.2) (end 55.37548 98.17548) (width 0.4) (layer "F.Cu") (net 1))
 (segment (start 56.75 102.2) (end 56.75 101.55) (width 0.4) (layer "F.Cu") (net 1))
 (segment (start 56.75 102.05) (end 57.6 101.2) (width 0.4) (layer "F.Cu") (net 1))
 (segment (start 56.083217 98.2) (end 55.4 98.2) (width 0.4) (layer "F.Cu") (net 1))
 (segment (start 60.6 100.45) (end 61 100.45) (width 0.4) (layer "F.Cu") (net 1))
 (segment (start 61 100.45) (end 62.7 98.75) (width 0.4) (layer "F.Cu") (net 1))
 (segment (start 57.6 101.2) (end 59.8 101.2) (width 0.4) (layer "F.Cu") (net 1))
 (segment (start 56.75 101.55) (end 55.6 100.4) (width 0.4) (layer "F.Cu") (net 1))
 (segment (start 55.37548 94.20048) (end 55 93.825) (width 0.4) (layer "F.Cu") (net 1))
 (segment (start 58.2 96.6) (end 58.2 97.223528) (width 0.4) (layer "F.Cu") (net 1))
 (segment (start 55.6 99.375) (end 56.6 98.375) (width 0.4) (layer "F.Cu") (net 1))
 (segment (start 58.2 97.223528) (end 57.048528 98.375) (width 0.4) (layer "F.Cu") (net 1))
 (segment (start 55.6 100.4) (end 55.6 99.375) (width 0.4) (layer "F.Cu") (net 1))
 (segment (start 51.768 93.4615) (end 54.6365 93.4615) (width 0.4) (layer "F.Cu") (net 1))
 (segment (start 55.052 104.2) (end 56.75 102.502) (width 0.4) (layer "F.Cu") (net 1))
 (segment (start 56.75 102.502) (end 56.75 102.2) (width 0.4) (layer "F.Cu") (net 1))
 (segment (start 55.37548 98.17548) (end 55.37548 94.20048) (width 0.4) (layer "F.Cu") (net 1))
 (segment (start 58.8 95.6) (end 58.8 96) (width 0.4) (layer "F.Cu") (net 1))
 (segment (start 59.8 101.2) (end 60.55 100.45) (width 0.4) (layer "F.Cu") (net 1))
 (segment (start 64.898 93.575) (end 66.15 94.827) (width 0.4) (layer "F.Cu") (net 4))
 (segment (start 66.15 94.827) (end 73.6435 94.827) (width 0.4) (layer "F.Cu") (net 4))
 (segment (start 62.7 92.65) (end 63.875 92.65) (width 0.4) (layer "F.Cu") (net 4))
 (segment (start 63.875 92.65) (end 64.8 93.575) (width 0.4) (layer "F.Cu") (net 4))
 (segment (start 73.6435 94.827) (end 75.009 93.4615) (width 0.4) (layer "F.Cu") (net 4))
 (segment (start 59.2 97) (end 59.654691 96.85) (width 0.25) (layer "F.Cu") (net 6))
 (segment (start 59.654691 96.85) (end 60.5 96.85) (width 0.25) (layer "F.Cu") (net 6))
 (via (at 59.2 97) (size 0.8) (drill 0.4) (layers "F.Cu" "B.Cu") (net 6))
 (via (at 56.8 93.7875) (size 0.8) (drill 0.4) (layers "F.Cu" "B.Cu") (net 6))
 (segment (start 59.2 96.036452) (end 56.8 93.7875) (width 0.25) (layer "B.Cu") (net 6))
 (segment (start 59.2 97) (end 59 96.8) (width 0.25) (layer "B.Cu") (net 6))
 (segment (start 59.2 97) (end 59.2 96.036452) (width 0.25) (layer "B.Cu") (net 6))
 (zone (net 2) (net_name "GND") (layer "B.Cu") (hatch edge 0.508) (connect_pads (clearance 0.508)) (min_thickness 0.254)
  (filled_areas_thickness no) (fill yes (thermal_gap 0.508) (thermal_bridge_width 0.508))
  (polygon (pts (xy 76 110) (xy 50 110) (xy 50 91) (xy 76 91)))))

